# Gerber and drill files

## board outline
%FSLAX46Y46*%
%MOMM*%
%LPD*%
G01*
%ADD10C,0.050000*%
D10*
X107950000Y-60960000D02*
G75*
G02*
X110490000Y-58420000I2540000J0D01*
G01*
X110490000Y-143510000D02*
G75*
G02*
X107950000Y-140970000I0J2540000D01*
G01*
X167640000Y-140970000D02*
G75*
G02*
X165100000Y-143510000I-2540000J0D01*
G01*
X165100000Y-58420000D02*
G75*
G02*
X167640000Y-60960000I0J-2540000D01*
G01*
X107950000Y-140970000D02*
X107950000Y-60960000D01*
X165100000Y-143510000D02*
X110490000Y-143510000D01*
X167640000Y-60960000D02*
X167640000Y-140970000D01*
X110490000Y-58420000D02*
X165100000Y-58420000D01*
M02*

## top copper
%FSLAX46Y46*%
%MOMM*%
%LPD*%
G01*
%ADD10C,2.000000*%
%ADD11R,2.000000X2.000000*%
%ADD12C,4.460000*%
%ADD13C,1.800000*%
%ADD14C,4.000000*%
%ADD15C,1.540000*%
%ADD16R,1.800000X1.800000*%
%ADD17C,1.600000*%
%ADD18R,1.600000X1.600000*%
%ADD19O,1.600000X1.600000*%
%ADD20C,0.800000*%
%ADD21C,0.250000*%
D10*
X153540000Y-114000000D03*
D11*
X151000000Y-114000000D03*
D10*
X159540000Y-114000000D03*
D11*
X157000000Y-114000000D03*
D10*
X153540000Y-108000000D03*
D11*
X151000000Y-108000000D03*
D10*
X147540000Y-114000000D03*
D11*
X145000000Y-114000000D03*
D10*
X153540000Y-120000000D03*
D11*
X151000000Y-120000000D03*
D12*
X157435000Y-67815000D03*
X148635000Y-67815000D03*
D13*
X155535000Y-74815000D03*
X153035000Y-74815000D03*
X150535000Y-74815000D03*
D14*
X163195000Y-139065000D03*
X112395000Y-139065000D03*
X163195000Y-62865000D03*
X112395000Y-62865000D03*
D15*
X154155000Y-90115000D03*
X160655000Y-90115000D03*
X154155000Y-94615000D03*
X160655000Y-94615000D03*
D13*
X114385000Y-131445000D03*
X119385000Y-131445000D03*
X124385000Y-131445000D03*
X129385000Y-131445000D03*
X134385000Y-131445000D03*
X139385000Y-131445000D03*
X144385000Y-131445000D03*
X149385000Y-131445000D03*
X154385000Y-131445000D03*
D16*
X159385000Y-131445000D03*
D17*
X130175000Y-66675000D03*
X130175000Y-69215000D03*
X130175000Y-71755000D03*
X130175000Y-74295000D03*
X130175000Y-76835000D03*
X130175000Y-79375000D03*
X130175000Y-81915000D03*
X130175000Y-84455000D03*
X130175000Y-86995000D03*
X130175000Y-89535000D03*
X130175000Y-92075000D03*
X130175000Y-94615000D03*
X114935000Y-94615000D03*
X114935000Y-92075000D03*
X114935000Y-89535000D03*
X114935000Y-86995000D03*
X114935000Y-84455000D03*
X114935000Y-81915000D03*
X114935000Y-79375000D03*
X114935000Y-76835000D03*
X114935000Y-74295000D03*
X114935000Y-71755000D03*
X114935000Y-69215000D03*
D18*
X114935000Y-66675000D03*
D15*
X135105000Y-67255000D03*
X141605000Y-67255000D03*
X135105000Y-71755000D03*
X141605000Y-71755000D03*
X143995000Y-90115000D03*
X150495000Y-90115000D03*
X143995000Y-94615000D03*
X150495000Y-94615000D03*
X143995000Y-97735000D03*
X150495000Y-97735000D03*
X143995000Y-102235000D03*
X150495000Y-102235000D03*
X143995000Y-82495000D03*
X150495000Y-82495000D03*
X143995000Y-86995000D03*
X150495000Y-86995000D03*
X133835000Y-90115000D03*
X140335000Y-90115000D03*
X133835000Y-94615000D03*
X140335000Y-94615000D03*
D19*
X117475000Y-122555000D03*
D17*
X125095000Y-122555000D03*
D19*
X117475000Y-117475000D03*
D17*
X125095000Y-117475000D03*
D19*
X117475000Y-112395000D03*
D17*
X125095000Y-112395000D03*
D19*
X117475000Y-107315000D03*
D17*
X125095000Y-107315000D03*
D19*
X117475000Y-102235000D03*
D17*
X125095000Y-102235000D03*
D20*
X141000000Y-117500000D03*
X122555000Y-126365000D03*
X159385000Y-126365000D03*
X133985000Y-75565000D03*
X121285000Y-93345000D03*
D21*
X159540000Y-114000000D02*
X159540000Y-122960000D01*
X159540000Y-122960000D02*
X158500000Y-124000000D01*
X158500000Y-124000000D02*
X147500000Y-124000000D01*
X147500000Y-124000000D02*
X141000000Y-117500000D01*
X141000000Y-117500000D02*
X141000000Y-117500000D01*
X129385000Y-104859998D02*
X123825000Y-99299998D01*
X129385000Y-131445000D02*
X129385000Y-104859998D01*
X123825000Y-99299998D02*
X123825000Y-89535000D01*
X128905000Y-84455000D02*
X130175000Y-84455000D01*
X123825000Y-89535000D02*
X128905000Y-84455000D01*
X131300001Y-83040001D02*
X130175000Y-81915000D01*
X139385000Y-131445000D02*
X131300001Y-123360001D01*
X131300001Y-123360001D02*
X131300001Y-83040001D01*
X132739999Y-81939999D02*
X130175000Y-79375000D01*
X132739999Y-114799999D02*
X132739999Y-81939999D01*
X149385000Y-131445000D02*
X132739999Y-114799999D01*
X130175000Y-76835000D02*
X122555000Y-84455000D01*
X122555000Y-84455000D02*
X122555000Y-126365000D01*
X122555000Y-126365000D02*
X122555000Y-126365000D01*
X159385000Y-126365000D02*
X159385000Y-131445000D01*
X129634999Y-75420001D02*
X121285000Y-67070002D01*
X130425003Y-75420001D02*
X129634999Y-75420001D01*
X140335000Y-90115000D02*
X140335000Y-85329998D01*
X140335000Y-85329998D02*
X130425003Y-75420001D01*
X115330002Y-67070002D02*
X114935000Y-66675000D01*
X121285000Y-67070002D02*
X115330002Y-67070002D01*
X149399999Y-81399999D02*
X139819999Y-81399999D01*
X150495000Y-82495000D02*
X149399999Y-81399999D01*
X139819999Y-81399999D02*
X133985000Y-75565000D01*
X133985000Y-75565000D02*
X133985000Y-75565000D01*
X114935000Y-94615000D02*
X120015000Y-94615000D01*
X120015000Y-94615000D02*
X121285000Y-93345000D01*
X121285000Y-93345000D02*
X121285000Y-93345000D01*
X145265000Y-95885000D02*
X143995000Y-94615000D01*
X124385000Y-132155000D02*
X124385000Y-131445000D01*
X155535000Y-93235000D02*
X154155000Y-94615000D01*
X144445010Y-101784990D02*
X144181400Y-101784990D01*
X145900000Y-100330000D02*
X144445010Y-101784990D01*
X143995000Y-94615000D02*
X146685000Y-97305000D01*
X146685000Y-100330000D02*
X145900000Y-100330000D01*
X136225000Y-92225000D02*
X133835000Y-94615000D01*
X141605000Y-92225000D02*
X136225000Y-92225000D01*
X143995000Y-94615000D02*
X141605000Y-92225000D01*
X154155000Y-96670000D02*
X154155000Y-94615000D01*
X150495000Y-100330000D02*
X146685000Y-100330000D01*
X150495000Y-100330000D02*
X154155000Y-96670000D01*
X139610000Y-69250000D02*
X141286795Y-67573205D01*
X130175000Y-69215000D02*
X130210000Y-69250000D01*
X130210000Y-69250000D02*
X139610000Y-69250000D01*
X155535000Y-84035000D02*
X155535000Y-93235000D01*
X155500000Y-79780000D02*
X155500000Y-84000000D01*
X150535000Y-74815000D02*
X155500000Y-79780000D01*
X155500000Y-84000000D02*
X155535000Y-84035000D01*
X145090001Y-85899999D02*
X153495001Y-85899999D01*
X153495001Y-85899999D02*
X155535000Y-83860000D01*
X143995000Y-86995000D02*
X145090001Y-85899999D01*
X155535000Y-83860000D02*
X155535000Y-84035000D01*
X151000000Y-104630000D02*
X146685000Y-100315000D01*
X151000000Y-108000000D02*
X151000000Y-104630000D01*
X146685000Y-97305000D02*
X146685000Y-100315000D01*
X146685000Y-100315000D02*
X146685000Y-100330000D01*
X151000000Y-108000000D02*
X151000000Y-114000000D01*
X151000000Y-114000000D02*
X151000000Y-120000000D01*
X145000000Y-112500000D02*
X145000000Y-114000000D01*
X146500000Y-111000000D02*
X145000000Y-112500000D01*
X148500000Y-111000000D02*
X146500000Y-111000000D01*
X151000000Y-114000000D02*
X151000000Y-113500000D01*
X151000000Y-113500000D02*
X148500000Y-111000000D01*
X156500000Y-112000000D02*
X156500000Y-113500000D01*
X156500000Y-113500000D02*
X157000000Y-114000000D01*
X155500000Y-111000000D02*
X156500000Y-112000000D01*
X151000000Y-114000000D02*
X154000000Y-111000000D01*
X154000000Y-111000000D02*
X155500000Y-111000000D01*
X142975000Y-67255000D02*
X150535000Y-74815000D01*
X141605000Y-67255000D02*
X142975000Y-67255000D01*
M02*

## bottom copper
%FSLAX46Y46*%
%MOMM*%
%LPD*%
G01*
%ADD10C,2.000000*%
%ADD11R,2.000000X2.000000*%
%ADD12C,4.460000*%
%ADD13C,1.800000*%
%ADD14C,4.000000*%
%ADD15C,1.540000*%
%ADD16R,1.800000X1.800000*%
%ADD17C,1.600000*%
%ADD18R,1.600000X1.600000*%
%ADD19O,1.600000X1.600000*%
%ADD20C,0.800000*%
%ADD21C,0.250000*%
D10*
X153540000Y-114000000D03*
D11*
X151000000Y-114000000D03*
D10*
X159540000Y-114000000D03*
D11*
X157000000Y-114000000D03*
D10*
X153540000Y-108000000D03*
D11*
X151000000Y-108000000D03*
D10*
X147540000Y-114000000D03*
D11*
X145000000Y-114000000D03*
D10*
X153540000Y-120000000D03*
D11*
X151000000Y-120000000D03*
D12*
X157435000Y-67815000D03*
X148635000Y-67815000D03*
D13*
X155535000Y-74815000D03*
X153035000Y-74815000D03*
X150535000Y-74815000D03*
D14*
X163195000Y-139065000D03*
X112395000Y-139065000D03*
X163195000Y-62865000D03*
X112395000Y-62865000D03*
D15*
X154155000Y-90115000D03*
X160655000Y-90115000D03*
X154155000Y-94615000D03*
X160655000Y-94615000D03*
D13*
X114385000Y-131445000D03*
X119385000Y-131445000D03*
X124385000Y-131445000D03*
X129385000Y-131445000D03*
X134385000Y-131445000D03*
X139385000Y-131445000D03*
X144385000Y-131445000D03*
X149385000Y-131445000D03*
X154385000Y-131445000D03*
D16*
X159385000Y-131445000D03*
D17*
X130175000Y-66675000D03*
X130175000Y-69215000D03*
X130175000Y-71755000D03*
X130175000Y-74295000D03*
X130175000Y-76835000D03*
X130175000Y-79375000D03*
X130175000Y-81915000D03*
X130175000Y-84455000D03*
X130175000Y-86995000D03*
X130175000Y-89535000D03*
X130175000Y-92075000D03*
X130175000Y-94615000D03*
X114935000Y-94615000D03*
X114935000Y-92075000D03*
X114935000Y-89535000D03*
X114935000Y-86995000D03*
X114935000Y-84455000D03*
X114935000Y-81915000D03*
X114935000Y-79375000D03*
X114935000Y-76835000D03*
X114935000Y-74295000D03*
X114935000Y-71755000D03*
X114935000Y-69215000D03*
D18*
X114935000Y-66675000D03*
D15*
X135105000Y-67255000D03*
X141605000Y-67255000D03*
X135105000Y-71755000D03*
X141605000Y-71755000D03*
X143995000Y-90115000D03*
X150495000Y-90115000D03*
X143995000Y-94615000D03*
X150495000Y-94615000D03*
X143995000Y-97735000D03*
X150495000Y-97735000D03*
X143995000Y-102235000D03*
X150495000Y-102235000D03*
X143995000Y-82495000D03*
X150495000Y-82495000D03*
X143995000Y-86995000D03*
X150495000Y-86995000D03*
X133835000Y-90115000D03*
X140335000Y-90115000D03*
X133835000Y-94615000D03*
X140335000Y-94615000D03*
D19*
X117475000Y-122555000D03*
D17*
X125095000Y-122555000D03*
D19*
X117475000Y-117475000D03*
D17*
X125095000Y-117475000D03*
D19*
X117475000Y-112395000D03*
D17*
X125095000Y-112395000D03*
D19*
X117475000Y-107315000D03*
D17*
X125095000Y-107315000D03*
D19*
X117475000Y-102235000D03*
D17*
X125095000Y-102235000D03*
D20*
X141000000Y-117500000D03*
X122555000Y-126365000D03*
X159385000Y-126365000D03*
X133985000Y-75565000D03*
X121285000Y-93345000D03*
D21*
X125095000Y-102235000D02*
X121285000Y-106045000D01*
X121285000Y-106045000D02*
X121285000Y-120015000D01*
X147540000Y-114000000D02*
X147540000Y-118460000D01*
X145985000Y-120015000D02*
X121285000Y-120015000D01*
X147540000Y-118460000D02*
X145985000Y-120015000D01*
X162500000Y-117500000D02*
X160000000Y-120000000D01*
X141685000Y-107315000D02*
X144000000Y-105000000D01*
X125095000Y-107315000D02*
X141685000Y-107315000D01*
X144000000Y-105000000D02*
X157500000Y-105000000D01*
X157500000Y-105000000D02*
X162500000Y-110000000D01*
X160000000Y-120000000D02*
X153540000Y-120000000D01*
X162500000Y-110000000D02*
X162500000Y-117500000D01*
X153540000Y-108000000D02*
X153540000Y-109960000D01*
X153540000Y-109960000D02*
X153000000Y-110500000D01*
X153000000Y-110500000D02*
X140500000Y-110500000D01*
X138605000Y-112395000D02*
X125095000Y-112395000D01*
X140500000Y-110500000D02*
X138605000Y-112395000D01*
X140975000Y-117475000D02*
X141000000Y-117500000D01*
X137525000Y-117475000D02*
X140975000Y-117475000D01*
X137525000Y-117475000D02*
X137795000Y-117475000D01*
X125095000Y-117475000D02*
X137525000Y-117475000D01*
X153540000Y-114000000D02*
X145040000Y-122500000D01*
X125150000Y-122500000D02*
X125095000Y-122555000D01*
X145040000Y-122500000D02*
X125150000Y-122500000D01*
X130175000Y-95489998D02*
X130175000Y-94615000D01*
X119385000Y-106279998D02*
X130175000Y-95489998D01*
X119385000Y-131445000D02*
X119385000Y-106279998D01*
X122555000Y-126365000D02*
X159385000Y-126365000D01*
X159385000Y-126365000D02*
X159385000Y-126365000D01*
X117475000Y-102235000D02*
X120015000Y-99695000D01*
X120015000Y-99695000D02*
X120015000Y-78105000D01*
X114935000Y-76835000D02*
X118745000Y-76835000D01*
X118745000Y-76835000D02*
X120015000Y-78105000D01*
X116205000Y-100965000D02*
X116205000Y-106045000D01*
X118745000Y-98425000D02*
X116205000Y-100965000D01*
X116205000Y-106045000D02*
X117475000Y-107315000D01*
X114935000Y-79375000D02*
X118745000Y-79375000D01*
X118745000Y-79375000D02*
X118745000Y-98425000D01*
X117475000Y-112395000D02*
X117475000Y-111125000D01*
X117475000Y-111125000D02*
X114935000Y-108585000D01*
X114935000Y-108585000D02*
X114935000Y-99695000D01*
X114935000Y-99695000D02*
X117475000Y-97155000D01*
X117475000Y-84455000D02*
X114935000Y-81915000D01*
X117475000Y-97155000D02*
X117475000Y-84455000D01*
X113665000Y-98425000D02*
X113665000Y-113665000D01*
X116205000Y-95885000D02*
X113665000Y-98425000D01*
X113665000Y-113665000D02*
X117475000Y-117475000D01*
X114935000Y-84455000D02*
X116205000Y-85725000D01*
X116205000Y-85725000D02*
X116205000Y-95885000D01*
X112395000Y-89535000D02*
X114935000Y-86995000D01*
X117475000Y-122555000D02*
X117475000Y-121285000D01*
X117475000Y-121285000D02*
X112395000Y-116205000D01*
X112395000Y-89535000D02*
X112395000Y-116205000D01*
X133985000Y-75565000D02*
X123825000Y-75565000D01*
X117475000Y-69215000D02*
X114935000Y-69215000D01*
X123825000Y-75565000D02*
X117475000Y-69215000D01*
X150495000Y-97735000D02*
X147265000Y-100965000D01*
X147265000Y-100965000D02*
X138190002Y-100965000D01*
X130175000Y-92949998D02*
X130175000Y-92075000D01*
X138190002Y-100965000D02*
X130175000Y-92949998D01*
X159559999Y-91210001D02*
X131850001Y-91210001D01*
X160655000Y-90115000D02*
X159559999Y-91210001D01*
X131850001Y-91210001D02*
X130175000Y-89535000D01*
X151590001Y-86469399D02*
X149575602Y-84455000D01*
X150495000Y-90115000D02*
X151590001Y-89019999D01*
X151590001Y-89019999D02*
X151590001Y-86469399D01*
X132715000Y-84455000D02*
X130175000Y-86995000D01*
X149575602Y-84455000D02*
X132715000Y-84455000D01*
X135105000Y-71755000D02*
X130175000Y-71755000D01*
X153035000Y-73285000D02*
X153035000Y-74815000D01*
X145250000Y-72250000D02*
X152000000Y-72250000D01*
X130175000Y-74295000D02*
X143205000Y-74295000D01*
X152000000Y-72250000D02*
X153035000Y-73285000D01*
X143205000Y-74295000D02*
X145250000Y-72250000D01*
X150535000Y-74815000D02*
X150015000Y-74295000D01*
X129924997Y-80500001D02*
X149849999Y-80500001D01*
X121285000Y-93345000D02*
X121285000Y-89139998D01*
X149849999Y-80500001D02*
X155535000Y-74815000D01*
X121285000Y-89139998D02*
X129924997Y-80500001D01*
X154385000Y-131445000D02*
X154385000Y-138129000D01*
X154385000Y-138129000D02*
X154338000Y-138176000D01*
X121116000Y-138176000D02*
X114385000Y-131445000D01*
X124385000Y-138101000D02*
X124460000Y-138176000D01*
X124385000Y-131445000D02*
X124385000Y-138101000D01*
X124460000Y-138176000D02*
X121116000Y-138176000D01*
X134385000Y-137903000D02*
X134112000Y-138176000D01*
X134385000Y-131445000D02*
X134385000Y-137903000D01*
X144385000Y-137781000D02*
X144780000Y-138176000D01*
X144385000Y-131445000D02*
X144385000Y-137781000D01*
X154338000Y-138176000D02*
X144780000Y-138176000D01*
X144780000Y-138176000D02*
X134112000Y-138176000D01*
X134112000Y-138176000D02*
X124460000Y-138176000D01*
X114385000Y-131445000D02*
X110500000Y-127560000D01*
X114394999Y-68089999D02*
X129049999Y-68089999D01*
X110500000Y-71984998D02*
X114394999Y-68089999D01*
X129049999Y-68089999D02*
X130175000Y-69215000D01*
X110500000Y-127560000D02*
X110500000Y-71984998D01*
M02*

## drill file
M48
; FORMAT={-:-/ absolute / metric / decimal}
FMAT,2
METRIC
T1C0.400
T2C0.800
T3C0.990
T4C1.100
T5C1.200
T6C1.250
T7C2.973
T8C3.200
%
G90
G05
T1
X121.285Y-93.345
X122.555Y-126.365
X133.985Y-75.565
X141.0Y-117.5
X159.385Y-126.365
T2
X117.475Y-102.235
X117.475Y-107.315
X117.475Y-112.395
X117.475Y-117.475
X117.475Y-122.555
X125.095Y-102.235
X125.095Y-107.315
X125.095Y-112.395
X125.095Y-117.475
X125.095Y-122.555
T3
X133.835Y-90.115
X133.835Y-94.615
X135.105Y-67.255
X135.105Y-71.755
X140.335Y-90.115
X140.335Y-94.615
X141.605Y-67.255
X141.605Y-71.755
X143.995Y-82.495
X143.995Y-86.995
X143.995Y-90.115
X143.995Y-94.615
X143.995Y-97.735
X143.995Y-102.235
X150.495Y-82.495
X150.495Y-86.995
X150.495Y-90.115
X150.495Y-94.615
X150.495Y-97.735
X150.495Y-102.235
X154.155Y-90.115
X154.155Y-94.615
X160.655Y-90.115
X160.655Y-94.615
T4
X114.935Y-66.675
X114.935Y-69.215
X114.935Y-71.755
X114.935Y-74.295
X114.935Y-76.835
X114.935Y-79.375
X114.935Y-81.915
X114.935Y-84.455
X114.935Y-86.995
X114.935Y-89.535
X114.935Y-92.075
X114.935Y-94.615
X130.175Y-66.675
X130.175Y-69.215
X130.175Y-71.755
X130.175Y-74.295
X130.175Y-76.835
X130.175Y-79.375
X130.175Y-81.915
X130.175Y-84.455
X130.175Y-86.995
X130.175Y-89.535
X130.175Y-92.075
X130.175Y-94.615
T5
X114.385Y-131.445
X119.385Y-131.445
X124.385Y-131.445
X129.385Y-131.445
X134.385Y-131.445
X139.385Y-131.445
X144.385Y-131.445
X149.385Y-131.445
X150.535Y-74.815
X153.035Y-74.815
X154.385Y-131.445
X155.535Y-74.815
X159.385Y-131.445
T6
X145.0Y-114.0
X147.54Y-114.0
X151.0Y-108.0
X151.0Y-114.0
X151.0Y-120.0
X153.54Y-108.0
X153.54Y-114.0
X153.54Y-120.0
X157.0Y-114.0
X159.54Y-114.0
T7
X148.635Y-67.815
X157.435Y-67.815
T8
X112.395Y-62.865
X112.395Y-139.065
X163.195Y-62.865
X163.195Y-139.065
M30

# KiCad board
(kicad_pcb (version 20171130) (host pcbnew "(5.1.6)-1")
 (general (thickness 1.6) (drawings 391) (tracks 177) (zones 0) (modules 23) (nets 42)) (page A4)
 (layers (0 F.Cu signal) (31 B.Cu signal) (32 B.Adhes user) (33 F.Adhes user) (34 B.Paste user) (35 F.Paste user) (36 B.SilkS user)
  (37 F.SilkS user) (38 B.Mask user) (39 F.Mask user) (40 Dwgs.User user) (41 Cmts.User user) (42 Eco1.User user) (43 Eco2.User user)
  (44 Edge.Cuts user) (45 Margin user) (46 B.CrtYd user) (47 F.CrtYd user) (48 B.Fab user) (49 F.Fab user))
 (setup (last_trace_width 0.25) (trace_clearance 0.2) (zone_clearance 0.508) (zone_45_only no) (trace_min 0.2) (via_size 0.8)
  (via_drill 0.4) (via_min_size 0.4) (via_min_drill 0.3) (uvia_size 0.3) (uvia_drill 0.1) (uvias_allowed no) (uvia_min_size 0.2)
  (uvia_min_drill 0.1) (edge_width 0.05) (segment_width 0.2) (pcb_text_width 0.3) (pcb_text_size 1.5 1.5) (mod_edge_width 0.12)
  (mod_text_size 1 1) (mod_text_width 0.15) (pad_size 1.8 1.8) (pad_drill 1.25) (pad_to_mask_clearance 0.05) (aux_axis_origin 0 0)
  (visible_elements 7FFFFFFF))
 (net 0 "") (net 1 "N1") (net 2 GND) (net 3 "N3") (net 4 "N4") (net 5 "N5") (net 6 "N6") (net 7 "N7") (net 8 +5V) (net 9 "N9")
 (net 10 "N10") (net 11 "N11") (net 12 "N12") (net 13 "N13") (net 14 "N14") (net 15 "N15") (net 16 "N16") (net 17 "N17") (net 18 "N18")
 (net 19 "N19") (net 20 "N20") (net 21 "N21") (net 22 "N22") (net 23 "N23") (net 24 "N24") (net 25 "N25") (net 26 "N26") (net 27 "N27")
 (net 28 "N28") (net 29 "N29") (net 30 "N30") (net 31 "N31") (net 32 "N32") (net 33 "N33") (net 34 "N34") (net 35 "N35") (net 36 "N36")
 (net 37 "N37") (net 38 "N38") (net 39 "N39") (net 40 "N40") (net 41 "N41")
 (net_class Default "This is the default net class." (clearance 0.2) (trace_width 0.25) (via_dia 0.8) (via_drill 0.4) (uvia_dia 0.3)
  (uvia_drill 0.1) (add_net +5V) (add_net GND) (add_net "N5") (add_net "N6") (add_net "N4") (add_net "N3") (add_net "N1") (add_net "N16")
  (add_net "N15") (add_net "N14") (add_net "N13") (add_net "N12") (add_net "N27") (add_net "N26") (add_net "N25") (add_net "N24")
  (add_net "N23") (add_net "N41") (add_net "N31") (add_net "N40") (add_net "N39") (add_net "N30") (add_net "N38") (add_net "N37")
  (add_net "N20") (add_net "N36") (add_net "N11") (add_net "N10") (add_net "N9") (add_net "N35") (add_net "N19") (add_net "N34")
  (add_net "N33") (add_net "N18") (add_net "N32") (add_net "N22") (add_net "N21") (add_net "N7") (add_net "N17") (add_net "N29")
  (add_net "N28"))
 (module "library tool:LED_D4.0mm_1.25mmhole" (layer F.Cu) (at 151 114)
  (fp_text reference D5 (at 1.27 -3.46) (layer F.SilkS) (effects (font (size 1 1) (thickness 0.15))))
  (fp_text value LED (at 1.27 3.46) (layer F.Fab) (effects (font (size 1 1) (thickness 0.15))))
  (pad 2 thru_hole circle (at 2.54 0) (size 2 2) (drill 1.25) (layers *.Cu *.Mask) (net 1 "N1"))
  (pad 1 thru_hole rect (at 0 0) (size 2 2) (drill 1.25) (layers *.Cu *.Mask) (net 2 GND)))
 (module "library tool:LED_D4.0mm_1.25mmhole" (layer F.Cu) (at 157 114)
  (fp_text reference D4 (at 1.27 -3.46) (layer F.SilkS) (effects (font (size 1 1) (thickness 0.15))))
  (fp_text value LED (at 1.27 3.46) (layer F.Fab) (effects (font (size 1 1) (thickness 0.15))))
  (pad 2 thru_hole circle (at 2.54 0) (size 2 2) (drill 1.25) (layers *.Cu *.Mask) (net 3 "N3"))
  (pad 1 thru_hole rect (at 0 0) (size 2 2) (drill 1.25) (layers *.Cu *.Mask) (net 2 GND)))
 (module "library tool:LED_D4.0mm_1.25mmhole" (layer F.Cu) (at 151 108)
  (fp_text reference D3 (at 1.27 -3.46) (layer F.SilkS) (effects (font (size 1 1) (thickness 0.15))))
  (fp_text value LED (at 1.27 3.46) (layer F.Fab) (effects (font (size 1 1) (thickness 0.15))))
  (pad 2 thru_hole circle (at 2.54 0) (size 2 2) (drill 1.25) (layers *.Cu *.Mask) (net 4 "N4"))
  (pad 1 thru_hole rect (at 0 0) (size 2 2) (drill 1.25) (layers *.Cu *.Mask) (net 2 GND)))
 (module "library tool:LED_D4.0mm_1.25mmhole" (layer F.Cu) (at 145 114)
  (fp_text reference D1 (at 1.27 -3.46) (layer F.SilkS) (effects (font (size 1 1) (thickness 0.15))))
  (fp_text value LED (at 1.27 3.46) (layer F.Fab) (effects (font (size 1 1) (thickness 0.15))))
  (pad 2 thru_hole circle (at 2.54 0) (size 2 2) (drill 1.25) (layers *.Cu *.Mask) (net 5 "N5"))
  (pad 1 thru_hole rect (at 0 0) (size 2 2) (drill 1.25) (layers *.Cu *.Mask) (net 2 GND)))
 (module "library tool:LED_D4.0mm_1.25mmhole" (layer F.Cu) (at 151 120)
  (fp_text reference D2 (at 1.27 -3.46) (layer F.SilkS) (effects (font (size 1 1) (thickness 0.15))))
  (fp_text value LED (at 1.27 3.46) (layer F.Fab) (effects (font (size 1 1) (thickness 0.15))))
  (pad 2 thru_hole circle (at 2.54 0) (size 2 2) (drill 1.25) (layers *.Cu *.Mask) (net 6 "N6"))
  (pad 1 thru_hole rect (at 0 0) (size 2 2) (drill 1.25) (layers *.Cu *.Mask) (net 2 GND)))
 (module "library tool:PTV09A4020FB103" (layer F.Cu) (at 153.035 69.215)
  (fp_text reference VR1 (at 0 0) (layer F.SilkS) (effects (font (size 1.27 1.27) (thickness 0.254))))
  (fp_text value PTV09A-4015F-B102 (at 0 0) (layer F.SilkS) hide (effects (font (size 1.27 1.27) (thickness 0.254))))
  (pad 5 thru_hole circle (at 4.4 -1.4) (size 4.46 4.46) (drill 2.9732) (layers *.Cu *.Mask))
  (pad 4 thru_hole circle (at -4.4 -1.4) (size 4.46 4.46) (drill 2.9732) (layers *.Cu *.Mask))
  (pad 3 thru_hole circle (at 2.5 5.6) (size 1.8 1.8) (drill 1.2) (layers *.Cu *.Mask) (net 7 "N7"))
  (pad 2 thru_hole circle (at 0 5.6) (size 1.8 1.8) (drill 1.2) (layers *.Cu *.Mask) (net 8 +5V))
  (pad 1 thru_hole circle (at -2.5 5.6) (size 1.8 1.8) (drill 1.2) (layers *.Cu *.Mask) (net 2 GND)))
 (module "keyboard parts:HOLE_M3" (layer F.Cu) (at 163.195 139.065 180)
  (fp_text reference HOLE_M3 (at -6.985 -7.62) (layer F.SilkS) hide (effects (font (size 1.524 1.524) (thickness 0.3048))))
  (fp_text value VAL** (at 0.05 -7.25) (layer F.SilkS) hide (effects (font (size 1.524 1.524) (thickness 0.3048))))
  (pad 1 thru_hole circle (at 0 0 180) (size 4 4) (drill 3.2) (layers *.Cu *.Mask F.SilkS)))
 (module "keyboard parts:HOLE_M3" (layer F.Cu) (at 112.395 139.065 90)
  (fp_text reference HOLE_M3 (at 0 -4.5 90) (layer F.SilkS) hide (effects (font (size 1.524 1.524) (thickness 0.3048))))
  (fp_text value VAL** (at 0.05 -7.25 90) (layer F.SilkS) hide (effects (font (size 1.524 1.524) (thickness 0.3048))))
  (pad 1 thru_hole circle (at 0 0 90) (size 4 4) (drill 3.2) (layers *.Cu *.Mask F.SilkS)))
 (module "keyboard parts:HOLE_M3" (layer F.Cu) (at 163.195 62.865 270)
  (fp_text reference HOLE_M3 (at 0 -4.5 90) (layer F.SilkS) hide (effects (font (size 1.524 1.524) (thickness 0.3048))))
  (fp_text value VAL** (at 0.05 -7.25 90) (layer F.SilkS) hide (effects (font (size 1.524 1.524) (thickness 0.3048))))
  (pad 1 thru_hole circle (at 0 0 270) (size 4 4) (drill 3.2) (layers *.Cu *.Mask F.SilkS)))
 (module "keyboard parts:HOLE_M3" (layer F.Cu) (at 112.395 62.865)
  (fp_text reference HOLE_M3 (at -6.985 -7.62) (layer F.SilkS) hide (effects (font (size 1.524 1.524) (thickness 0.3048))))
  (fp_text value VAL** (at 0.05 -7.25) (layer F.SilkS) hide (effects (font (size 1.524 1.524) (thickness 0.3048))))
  (pad 1 thru_hole circle (at 0 0) (size 4 4) (drill 3.2) (layers *.Cu *.Mask F.SilkS)))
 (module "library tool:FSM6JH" (layer F.Cu) (at 160.655 94.615)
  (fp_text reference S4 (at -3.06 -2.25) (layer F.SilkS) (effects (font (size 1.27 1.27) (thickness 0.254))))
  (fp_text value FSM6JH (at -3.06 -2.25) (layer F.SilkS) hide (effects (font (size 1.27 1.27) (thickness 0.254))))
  (pad 4 thru_hole circle (at -6.5 -4.5) (size 1.54 1.54) (drill 0.99) (layers *.Cu *.Mask) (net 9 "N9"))
  (pad 3 thru_hole circle (at 0 -4.5) (size 1.54 1.54) (drill 0.99) (layers *.Cu *.Mask) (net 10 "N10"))
  (pad 2 thru_hole circle (at -6.5 0) (size 1.54 1.54) (drill 0.99) (layers *.Cu *.Mask) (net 2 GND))
  (pad 1 thru_hole circle (at 0 0) (size 1.54 1.54) (drill 0.99) (layers *.Cu *.Mask) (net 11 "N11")))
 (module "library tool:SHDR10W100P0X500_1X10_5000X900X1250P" (layer F.Cu) (at 159.385 131.445 180)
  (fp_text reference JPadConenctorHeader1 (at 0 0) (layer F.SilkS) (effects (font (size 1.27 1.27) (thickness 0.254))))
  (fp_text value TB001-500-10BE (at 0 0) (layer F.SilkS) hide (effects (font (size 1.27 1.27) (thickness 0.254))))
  (pad 10 thru_hole circle (at 45 0 180) (size 1.8 1.8) (drill 1.2) (layers *.Cu *.Mask) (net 2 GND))
  (pad 9 thru_hole circle (at 40 0 180) (size 1.8 1.8) (drill 1.2) (layers *.Cu *.Mask) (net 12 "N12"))
  (pad 8 thru_hole circle (at 35 0 180) (size 1.8 1.8) (drill 1.2) (layers *.Cu *.Mask) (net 2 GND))
  (pad 7 thru_hole circle (at 30 0 180) (size 1.8 1.8) (drill 1.2) (layers *.Cu *.Mask) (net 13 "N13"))
  (pad 6 thru_hole circle (at 25 0 180) (size 1.8 1.8) (drill 1.2) (layers *.Cu *.Mask) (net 2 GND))
  (pad 5 thru_hole circle (at 20 0 180) (size 1.8 1.8) (drill 1.2) (layers *.Cu *.Mask) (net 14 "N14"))
  (pad 4 thru_hole circle (at 15 0 180) (size 1.8 1.8) (drill 1.2) (layers *.Cu *.Mask) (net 2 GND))
  (pad 3 thru_hole circle (at 10 0 180) (size 1.8 1.8) (drill 1.2) (layers *.Cu *.Mask) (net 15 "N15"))
  (pad 2 thru_hole circle (at 5 0 180) (size 1.8 1.8) (drill 1.2) (layers *.Cu *.Mask) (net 2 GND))
  (pad 1 thru_hole rect (at 0 0 180) (size 1.8 1.8) (drill 1.2) (layers *.Cu *.Mask) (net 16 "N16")))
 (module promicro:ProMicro (layer F.Cu) (at 122.555 80.645 270)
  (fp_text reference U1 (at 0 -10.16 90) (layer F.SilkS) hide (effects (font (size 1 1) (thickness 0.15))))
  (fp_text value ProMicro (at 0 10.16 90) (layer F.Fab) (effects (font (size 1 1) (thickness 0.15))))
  (pad 24 thru_hole circle (at -13.97 -7.62 270) (size 1.6 1.6) (drill 1.1) (layers *.Cu *.Mask F.SilkS) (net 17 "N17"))
  (pad 23 thru_hole circle (at -11.43 -7.62 270) (size 1.6 1.6) (drill 1.1) (layers *.Cu *.Mask F.SilkS) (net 2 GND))
  (pad 22 thru_hole circle (at -8.89 -7.62 270) (size 1.6 1.6) (drill 1.1) (layers *.Cu *.Mask F.SilkS) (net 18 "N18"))
  (pad 21 thru_hole circle (at -6.35 -7.62 270) (size 1.6 1.6) (drill 1.1) (layers *.Cu *.Mask F.SilkS) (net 8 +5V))
  (pad 20 thru_hole circle (at -3.81 -7.62 270) (size 1.6 1.6) (drill 1.1) (layers *.Cu *.Mask F.SilkS) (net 16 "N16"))
  (pad 19 thru_hole circle (at -1.27 -7.62 270) (size 1.6 1.6) (drill 1.1) (layers *.Cu *.Mask F.SilkS) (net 15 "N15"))
  (pad 18 thru_hole circle (at 1.27 -7.62 270) (size 1.6 1.6) (drill 1.1) (layers *.Cu *.Mask F.SilkS) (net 14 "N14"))
  (pad 17 thru_hole circle (at 3.81 -7.62 270) (size 1.6 1.6) (drill 1.1) (layers *.Cu *.Mask F.SilkS) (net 13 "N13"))
  (pad 16 thru_hole circle (at 6.35 -7.62 270) (size 1.6 1.6) (drill 1.1) (layers *.Cu *.Mask F.SilkS) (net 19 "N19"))
  (pad 15 thru_hole circle (at 8.89 -7.62 270) (size 1.6 1.6) (drill 1.1) (layers *.Cu *.Mask F.SilkS) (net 10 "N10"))
  (pad 14 thru_hole circle (at 11.43 -7.62 270) (size 1.6 1.6) (drill 1.1) (layers *.Cu *.Mask F.SilkS) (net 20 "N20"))
  (pad 13 thru_hole circle (at 13.97 -7.62 270) (size 1.6 1.6) (drill 1.1) (layers *.Cu *.Mask F.SilkS) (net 12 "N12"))
  (pad 12 thru_hole circle (at 13.97 7.62 270) (size 1.6 1.6) (drill 1.1) (layers *.Cu *.Mask F.SilkS) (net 7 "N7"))
  (pad 11 thru_hole circle (at 11.43 7.62 270) (size 1.6 1.6) (drill 1.1) (layers *.Cu *.Mask F.SilkS) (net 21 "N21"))
  (pad 10 thru_hole circle (at 8.89 7.62 270) (size 1.6 1.6) (drill 1.1) (layers *.Cu *.Mask F.SilkS) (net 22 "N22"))
  (pad 9 thru_hole circle (at 6.35 7.62 270) (size 1.6 1.6) (drill 1.1) (layers *.Cu *.Mask F.SilkS) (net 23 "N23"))
  (pad 8 thru_hole circle (at 3.81 7.62 270) (size 1.6 1.6) (drill 1.1) (layers *.Cu *.Mask F.SilkS) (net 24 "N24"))
  (pad 7 thru_hole circle (at 1.27 7.62 270) (size 1.6 1.6) (drill 1.1) (layers *.Cu *.Mask F.SilkS) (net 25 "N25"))
  (pad 6 thru_hole circle (at -1.27 7.62 270) (size 1.6 1.6) (drill 1.1) (layers *.Cu *.Mask F.SilkS) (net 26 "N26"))
  (pad 5 thru_hole circle (at -3.81 7.62 270) (size 1.6 1.6) (drill 1.1) (layers *.Cu *.Mask F.SilkS) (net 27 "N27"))
  (pad 4 thru_hole circle (at -6.35 7.62 270) (size 1.6 1.6) (drill 1.1) (layers *.Cu *.Mask F.SilkS) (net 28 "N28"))
  (pad 3 thru_hole circle (at -8.89 7.62 270) (size 1.6 1.6) (drill 1.1) (layers *.Cu *.Mask F.SilkS) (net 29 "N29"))
  (pad 2 thru_hole circle (at -11.43 7.62 270) (size 1.6 1.6) (drill 1.1) (layers *.Cu *.Mask F.SilkS) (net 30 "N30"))
  (pad 1 thru_hole rect (at -13.97 7.62 270) (size 1.6 1.6) (drill 1.1) (layers *.Cu *.Mask F.SilkS) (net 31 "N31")))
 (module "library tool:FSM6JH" (layer F.Cu) (at 141.605 71.755)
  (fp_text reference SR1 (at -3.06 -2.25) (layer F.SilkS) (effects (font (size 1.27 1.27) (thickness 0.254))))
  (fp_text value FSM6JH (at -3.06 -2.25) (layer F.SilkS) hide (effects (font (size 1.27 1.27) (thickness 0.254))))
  (pad 4 thru_hole circle (at -6.5 -4.5) (size 1.54 1.54) (drill 0.99) (layers *.Cu *.Mask) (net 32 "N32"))
  (pad 3 thru_hole circle (at 0 -4.5) (size 1.54 1.54) (drill 0.99) (layers *.Cu *.Mask) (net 2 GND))
  (pad 2 thru_hole circle (at -6.5 0) (size 1.54 1.54) (drill 0.99) (layers *.Cu *.Mask) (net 18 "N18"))
  (pad 1 thru_hole circle (at 0 0) (size 1.54 1.54) (drill 0.99) (layers *.Cu *.Mask) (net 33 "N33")))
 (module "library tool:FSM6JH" (layer F.Cu) (at 150.495 94.615)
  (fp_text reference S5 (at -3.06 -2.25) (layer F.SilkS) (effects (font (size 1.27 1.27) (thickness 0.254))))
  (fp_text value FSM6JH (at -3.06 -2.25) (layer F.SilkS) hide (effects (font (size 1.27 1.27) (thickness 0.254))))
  (pad 4 thru_hole circle (at -6.5 -4.5) (size 1.54 1.54) (drill 0.99) (layers *.Cu *.Mask) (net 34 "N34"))
  (pad 3 thru_hole circle (at 0 -4.5) (size 1.54 1.54) (drill 0.99) (layers *.Cu *.Mask) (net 19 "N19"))
  (pad 2 thru_hole circle (at -6.5 0) (size 1.54 1.54) (drill 0.99) (layers *.Cu *.Mask) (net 2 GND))
  (pad 1 thru_hole circle (at 0 0) (size 1.54 1.54) (drill 0.99) (layers *.Cu *.Mask) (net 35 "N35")))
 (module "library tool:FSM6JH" (layer F.Cu) (at 150.495 102.235)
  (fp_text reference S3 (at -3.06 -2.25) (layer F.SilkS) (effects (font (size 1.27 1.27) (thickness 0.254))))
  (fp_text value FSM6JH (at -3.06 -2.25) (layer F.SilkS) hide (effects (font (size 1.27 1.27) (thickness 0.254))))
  (pad 4 thru_hole circle (at -6.5 -4.5) (size 1.54 1.54) (drill 0.99) (layers *.Cu *.Mask) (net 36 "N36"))
  (pad 3 thru_hole circle (at 0 -4.5) (size 1.54 1.54) (drill 0.99) (layers *.Cu *.Mask) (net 20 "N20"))
  (pad 2 thru_hole circle (at -6.5 0) (size 1.54 1.54) (drill 0.99) (layers *.Cu *.Mask) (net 2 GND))
  (pad 1 thru_hole circle (at 0 0) (size 1.54 1.54) (drill 0.99) (layers *.Cu *.Mask) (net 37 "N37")))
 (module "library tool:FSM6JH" (layer F.Cu) (at 150.495 86.995)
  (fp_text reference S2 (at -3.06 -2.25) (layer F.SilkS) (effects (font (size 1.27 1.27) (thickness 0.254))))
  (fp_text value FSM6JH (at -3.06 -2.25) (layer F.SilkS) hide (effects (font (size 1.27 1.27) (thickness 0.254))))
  (pad 4 thru_hole circle (at -6.5 -4.5) (size 1.54 1.54) (drill 0.99) (layers *.Cu *.Mask) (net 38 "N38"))
  (pad 3 thru_hole circle (at 0 -4.5) (size 1.54 1.54) (drill 0.99) (layers *.Cu *.Mask) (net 30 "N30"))
  (pad 2 thru_hole circle (at -6.5 0) (size 1.54 1.54) (drill 0.99) (layers *.Cu *.Mask) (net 2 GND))
  (pad 1 thru_hole circle (at 0 0) (size 1.54 1.54) (drill 0.99) (layers *.Cu *.Mask) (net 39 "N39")))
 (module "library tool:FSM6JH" (layer F.Cu) (at 140.335 94.615)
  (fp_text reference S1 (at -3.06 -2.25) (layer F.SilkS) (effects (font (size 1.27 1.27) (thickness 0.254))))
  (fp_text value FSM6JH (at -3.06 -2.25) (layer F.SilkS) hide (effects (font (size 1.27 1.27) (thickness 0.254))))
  (pad 4 thru_hole circle (at -6.5 -4.5) (size 1.54 1.54) (drill 0.99) (layers *.Cu *.Mask) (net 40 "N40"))
  (pad 3 thru_hole circle (at 0 -4.5) (size 1.54 1.54) (drill 0.99) (layers *.Cu *.Mask) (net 31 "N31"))
  (pad 2 thru_hole circle (at -6.5 0) (size 1.54 1.54) (drill 0.99) (layers *.Cu *.Mask) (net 2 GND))
  (pad 1 thru_hole circle (at 0 0) (size 1.54 1.54) (drill 0.99) (layers *.Cu *.Mask) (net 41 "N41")))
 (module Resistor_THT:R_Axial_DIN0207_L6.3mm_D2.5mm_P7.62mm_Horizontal (layer F.Cu) (at 125.095 122.555 180)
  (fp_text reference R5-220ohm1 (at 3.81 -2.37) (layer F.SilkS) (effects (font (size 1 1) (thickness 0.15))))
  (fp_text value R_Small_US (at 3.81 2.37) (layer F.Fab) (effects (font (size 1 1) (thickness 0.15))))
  (pad 2 thru_hole oval (at 7.62 0 180) (size 1.6 1.6) (drill 0.8) (layers *.Cu *.Mask) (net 23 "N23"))
  (pad 1 thru_hole circle (at 0 0 180) (size 1.6 1.6) (drill 0.8) (layers *.Cu *.Mask) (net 1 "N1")))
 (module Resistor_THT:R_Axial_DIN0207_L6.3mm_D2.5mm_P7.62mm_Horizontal (layer F.Cu) (at 125.095 117.475 180)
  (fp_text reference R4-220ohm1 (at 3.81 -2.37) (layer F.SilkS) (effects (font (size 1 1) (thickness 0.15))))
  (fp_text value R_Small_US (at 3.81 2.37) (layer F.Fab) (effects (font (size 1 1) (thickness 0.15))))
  (pad 2 thru_hole oval (at 7.62 0 180) (size 1.6 1.6) (drill 0.8) (layers *.Cu *.Mask) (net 24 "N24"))
  (pad 1 thru_hole circle (at 0 0 180) (size 1.6 1.6) (drill 0.8) (layers *.Cu *.Mask) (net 3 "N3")))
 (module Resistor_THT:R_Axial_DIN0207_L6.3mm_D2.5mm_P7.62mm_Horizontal (layer F.Cu) (at 125.095 112.395 180)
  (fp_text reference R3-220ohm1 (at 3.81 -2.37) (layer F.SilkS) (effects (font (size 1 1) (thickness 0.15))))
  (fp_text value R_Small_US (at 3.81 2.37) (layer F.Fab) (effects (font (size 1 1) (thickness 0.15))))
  (pad 2 thru_hole oval (at 7.62 0 180) (size 1.6 1.6) (drill 0.8) (layers *.Cu *.Mask) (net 25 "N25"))
  (pad 1 thru_hole circle (at 0 0 180) (size 1.6 1.6) (drill 0.8) (layers *.Cu *.Mask) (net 4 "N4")))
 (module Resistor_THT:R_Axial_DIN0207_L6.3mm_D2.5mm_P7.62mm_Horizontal (layer F.Cu) (at 125.095 107.315 180)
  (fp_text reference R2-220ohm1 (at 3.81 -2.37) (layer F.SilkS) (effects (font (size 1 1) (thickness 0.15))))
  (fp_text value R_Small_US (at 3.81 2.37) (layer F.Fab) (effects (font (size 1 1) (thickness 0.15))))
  (pad 2 thru_hole oval (at 7.62 0 180) (size 1.6 1.6) (drill 0.8) (layers *.Cu *.Mask) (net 26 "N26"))
  (pad 1 thru_hole circle (at 0 0 180) (size 1.6 1.6) (drill 0.8) (layers *.Cu *.Mask) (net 6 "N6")))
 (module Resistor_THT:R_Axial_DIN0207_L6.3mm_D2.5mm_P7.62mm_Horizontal (layer F.Cu) (at 125.095 102.235 180)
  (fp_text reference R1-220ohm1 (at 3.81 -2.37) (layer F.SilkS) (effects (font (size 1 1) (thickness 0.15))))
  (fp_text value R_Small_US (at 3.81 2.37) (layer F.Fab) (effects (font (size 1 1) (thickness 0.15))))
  (pad 2 thru_hole oval (at 7.62 0 180) (size 1.6 1.6) (drill 0.8) (layers *.Cu *.Mask) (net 27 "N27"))
  (pad 1 thru_hole circle (at 0 0 180) (size 1.6 1.6) (drill 0.8) (layers *.Cu *.Mask) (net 5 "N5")))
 (gr_arc (start 110.49 60.96) (end 110.49 58.42) (angle -90) (layer Edge.Cuts) (width 0.05))
 (gr_arc (start 110.49 140.97) (end 107.95 140.97) (angle -90) (layer Edge.Cuts) (width 0.05))
 (gr_arc (start 165.1 140.97) (end 165.1 143.51) (angle -90) (layer Edge.Cuts) (width 0.05))
 (gr_arc (start 165.1 60.96) (end 167.64 60.96) (angle -90) (layer Edge.Cuts) (width 0.05))
 (gr_line (start 107.95 140.97) (end 107.95 60.96) (layer Edge.Cuts) (width 0.05))
 (gr_line (start 165.1 143.51) (end 110.49 143.51) (layer Edge.Cuts) (width 0.05))
 (gr_line (start 167.64 60.96) (end 167.64 140.97) (layer Edge.Cuts) (width 0.05))
 (gr_line (start 110.49 58.42) (end 165.1 58.42) (layer Edge.Cuts) (width 0.05))
 (segment (start 125.095 102.235) (end 121.285 106.045) (width 0.25) (layer B.Cu) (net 5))
 (segment (start 121.285 106.045) (end 121.285 120.015) (width 0.25) (layer B.Cu) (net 5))
 (segment (start 147.54 114) (end 147.54 118.46) (width 0.25) (layer B.Cu) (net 5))
 (segment (start 145.985 120.015) (end 121.285 120.015) (width 0.25) (layer B.Cu) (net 5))
 (segment (start 147.54 118.46) (end 145.985 120.015) (width 0.25) (layer B.Cu) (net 5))
 (segment (start 162.5 117.5) (end 160 120) (width 0.25) (layer B.Cu) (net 6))
 (segment (start 141.685 107.315) (end 144 105) (width 0.25) (layer B.Cu) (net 6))
 (segment (start 125.095 107.315) (end 141.685 107.315) (width 0.25) (layer B.Cu) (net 6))
 (segment (start 144 105) (end 157.5 105) (width 0.25) (layer B.Cu) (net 6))
 (segment (start 157.5 105) (end 162.5 110) (width 0.25) (layer B.Cu) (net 6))
 (segment (start 160 120) (end 153.54 120) (width 0.25) (layer B.Cu) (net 6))
 (segment (start 162.5 110) (end 162.5 117.5) (width 0.25) (layer B.Cu) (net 6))
 (segment (start 153.54 108) (end 153.54 109.96) (width 0.25) (layer B.Cu) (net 4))
 (segment (start 153.54 109.96) (end 153 110.5) (width 0.25) (layer B.Cu) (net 4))
 (segment (start 153 110.5) (end 140.5 110.5) (width 0.25) (layer B.Cu) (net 4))
 (segment (start 138.605 112.395) (end 125.095 112.395) (width 0.25) (layer B.Cu) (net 4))
 (segment (start 140.5 110.5) (end 138.605 112.395) (width 0.25) (layer B.Cu) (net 4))
 (segment (start 159.54 114) (end 159.54 122.96) (width 0.25) (layer F.Cu) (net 3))
 (segment (start 159.54 122.96) (end 158.5 124) (width 0.25) (layer F.Cu) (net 3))
 (segment (start 158.5 124) (end 147.5 124) (width 0.25) (layer F.Cu) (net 3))
 (segment (start 147.5 124) (end 141 117.5) (width 0.25) (layer F.Cu) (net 3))
 (segment (start 141 117.5) (end 141 117.5) (width 0.25) (layer F.Cu) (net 3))
 (via (at 141 117.5) (size 0.8) (drill 0.4) (layers F.Cu B.Cu) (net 3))
 (segment (start 140.975 117.475) (end 141 117.5) (width 0.25) (layer B.Cu) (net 3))
 (segment (start 137.525 117.475) (end 140.975 117.475) (width 0.25) (layer B.Cu) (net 3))
 (segment (start 137.525 117.475) (end 137.795 117.475) (width 0.25) (layer B.Cu) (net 3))
 (segment (start 125.095 117.475) (end 137.525 117.475) (width 0.25) (layer B.Cu) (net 3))
 (segment (start 153.54 114) (end 145.04 122.5) (width 0.25) (layer B.Cu) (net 1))
 (segment (start 125.15 122.5) (end 125.095 122.555) (width 0.25) (layer B.Cu) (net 1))
 (segment (start 145.04 122.5) (end 125.15 122.5) (width 0.25) (layer B.Cu) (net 1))
 (segment (start 130.175 95.489998) (end 130.175 94.615) (width 0.25) (layer B.Cu) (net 12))
 (segment (start 119.385 106.279998) (end 130.175 95.489998) (width 0.25) (layer B.Cu) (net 12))
 (segment (start 119.385 131.445) (end 119.385 106.279998) (width 0.25) (layer B.Cu) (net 12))
 (segment (start 129.385 104.859998) (end 123.825 99.299998) (width 0.25) (layer F.Cu) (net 13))
 (segment (start 129.385 131.445) (end 129.385 104.859998) (width 0.25) (layer F.Cu) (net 13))
 (segment (start 123.825 99.299998) (end 123.825 89.535) (width 0.25) (layer F.Cu) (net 13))
 (segment (start 128.905 84.455) (end 130.175 84.455) (width 0.25) (layer F.Cu) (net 13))
 (segment (start 123.825 89.535) (end 128.905 84.455) (width 0.25) (layer F.Cu) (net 13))
 (segment (start 131.300001 83.040001) (end 130.175 81.915) (width 0.25) (layer F.Cu) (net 14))
 (segment (start 139.385 131.445) (end 131.300001 123.360001) (width 0.25) (layer F.Cu) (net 14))
 (segment (start 131.300001 123.360001) (end 131.300001 83.040001) (width 0.25) (layer F.Cu) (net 14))
 (segment (start 132.739999 81.939999) (end 130.175 79.375) (width 0.25) (layer F.Cu) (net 15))
 (segment (start 132.739999 114.799999) (end 132.739999 81.939999) (width 0.25) (layer F.Cu) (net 15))
 (segment (start 149.385 131.445) (end 132.739999 114.799999) (width 0.25) (layer F.Cu) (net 15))
 (segment (start 130.175 76.835) (end 122.555 84.455) (width 0.25) (layer F.Cu) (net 16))
 (segment (start 122.555 84.455) (end 122.555 126.365) (width 0.25) (layer F.Cu) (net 16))
 (segment (start 122.555 126.365) (end 122.555 126.365) (width 0.25) (layer F.Cu) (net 16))
 (via (at 122.555 126.365) (size 0.8) (drill 0.4) (layers F.Cu B.Cu) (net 16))
 (segment (start 122.555 126.365) (end 159.385 126.365) (width 0.25) (layer B.Cu) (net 16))
 (segment (start 159.385 126.365) (end 159.385 126.365) (width 0.25) (layer B.Cu) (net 16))
 (via (at 159.385 126.365) (size 0.8) (drill 0.4) (layers F.Cu B.Cu) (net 16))
 (segment (start 159.385 126.365) (end 159.385 131.445) (width 0.25) (layer F.Cu) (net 16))
 (segment (start 117.475 102.235) (end 120.015 99.695) (width 0.25) (layer B.Cu) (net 27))
 (segment (start 120.015 99.695) (end 120.015 78.105) (width 0.25) (layer B.Cu) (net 27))
 (segment (start 114.935 76.835) (end 118.745 76.835) (width 0.25) (layer B.Cu) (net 27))
 (segment (start 118.745 76.835) (end 120.015 78.105) (width 0.25) (layer B.Cu) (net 27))
 (segment (start 116.205 100.965) (end 116.205 106.045) (width 0.25) (layer B.Cu) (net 26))
 (segment (start 118.745 98.425) (end 116.205 100.965) (width 0.25) (layer B.Cu) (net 26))
 (segment (start 116.205 106.045) (end 117.475 107.315) (width 0.25) (layer B.Cu) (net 26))
 (segment (start 114.935 79.375) (end 118.745 79.375) (width 0.25) (layer B.Cu) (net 26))
 (segment (start 118.745 79.375) (end 118.745 98.425) (width 0.25) (layer B.Cu) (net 26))
 (segment (start 117.475 112.395) (end 117.475 111.125) (width 0.25) (layer B.Cu) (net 25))
 (segment (start 117.475 111.125) (end 114.935 108.585) (width 0.25) (layer B.Cu) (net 25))
 (segment (start 114.935 108.585) (end 114.935 99.695) (width 0.25) (layer B.Cu) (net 25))
 (segment (start 114.935 99.695) (end 117.475 97.155) (width 0.25) (layer B.Cu) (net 25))
 (segment (start 117.475 84.455) (end 114.935 81.915) (width 0.25) (layer B.Cu) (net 25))
 (segment (start 117.475 97.155) (end 117.475 84.455) (width 0.25) (layer B.Cu) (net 25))
 (segment (start 113.665 98.425) (end 113.665 113.665) (width 0.25) (layer B.Cu) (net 24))
 (segment (start 116.205 95.885) (end 113.665 98.425) (width 0.25) (layer B.Cu) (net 24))
 (segment (start 113.665 113.665) (end 117.475 117.475) (width 0.25) (layer B.Cu) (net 24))
 (segment (start 114.935 84.455) (end 116.205 85.725) (width 0.25) (layer B.Cu) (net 24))
 (segment (start 116.205 85.725) (end 116.205 95.885) (width 0.25) (layer B.Cu) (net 24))
 (segment (start 112.395 89.535) (end 114.935 86.995) (width 0.25) (layer B.Cu) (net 23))
 (segment (start 117.475 122.555) (end 117.475 121.285) (width 0.25) (layer B.Cu) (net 23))
 (segment (start 117.475 121.285) (end 112.395 116.205) (width 0.25) (layer B.Cu) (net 23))
 (segment (start 112.395 89.535) (end 112.395 116.205) (width 0.25) (layer B.Cu) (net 23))
 (segment (start 129.634999 75.420001) (end 121.285 67.070002) (width 0.25) (layer F.Cu) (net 31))
 (segment (start 130.425003 75.420001) (end 129.634999 75.420001) (width 0.25) (layer F.Cu) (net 31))
 (segment (start 140.335 90.115) (end 140.335 85.329998) (width 0.25) (layer F.Cu) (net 31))
 (segment (start 140.335 85.329998) (end 130.425003 75.420001) (width 0.25) (layer F.Cu) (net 31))
 (segment (start 115.330002 67.070002) (end 114.935 66.675) (width 0.25) (layer F.Cu) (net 31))
 (segment (start 121.285 67.070002) (end 115.330002 67.070002) (width 0.25) (layer F.Cu) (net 31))
 (segment (start 149.399999 81.399999) (end 139.819999 81.399999) (width 0.25) (layer F.Cu) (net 30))
 (segment (start 150.495 82.495) (end 149.399999 81.399999) (width 0.25) (layer F.Cu) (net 30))
 (segment (start 139.819999 81.399999) (end 133.985 75.565) (width 0.25) (layer F.Cu) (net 30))
 (segment (start 133.985 75.565) (end 133.985 75.565) (width 0.25) (layer F.Cu) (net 30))
 (via (at 133.985 75.565) (size 0.8) (drill 0.4) (layers F.Cu B.Cu) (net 30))
 (segment (start 133.985 75.565) (end 123.825 75.565) (width 0.25) (layer B.Cu) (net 30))
 (segment (start 117.475 69.215) (end 114.935 69.215) (width 0.25) (layer B.Cu) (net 30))
 (segment (start 123.825 75.565) (end 117.475 69.215) (width 0.25) (layer B.Cu) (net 30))
 (segment (start 150.495 97.735) (end 147.265 100.965) (width 0.25) (layer B.Cu) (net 20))
 (segment (start 147.265 100.965) (end 138.190002 100.965) (width 0.25) (layer B.Cu) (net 20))
 (segment (start 130.175 92.949998) (end 130.175 92.075) (width 0.25) (layer B.Cu) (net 20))
 (segment (start 138.190002 100.965) (end 130.175 92.949998) (width 0.25) (layer B.Cu) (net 20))
 (segment (start 159.559999 91.210001) (end 131.850001 91.210001) (width 0.25) (layer B.Cu) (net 10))
 (segment (start 160.655 90.115) (end 159.559999 91.210001) (width 0.25) (layer B.Cu) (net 10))
 (segment (start 131.850001 91.210001) (end 130.175 89.535) (width 0.25) (layer B.Cu) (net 10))
 (segment (start 151.590001 86.469399) (end 149.575602 84.455) (width 0.25) (layer B.Cu) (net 19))
 (segment (start 150.495 90.115) (end 151.590001 89.019999) (width 0.25) (layer B.Cu) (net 19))
 (segment (start 151.590001 89.019999) (end 151.590001 86.469399) (width 0.25) (layer B.Cu) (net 19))
 (segment (start 132.715 84.455) (end 130.175 86.995) (width 0.25) (layer B.Cu) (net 19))
 (segment (start 149.575602 84.455) (end 132.715 84.455) (width 0.25) (layer B.Cu) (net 19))
 (segment (start 135.105 71.755) (end 130.175 71.755) (width 0.25) (layer B.Cu) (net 18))
 (segment (start 153.035 73.285) (end 153.035 74.815) (width 0.25) (layer B.Cu) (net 8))
 (segment (start 145.25 72.25) (end 152 72.25) (width 0.25) (layer B.Cu) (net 8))
 (segment (start 130.175 74.295) (end 143.205 74.295) (width 0.25) (layer B.Cu) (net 8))
 (segment (start 152 72.25) (end 153.035 73.285) (width 0.25) (layer B.Cu) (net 8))
 (segment (start 143.205 74.295) (end 145.25 72.25) (width 0.25) (layer B.Cu) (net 8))
 (segment (start 150.535 74.815) (end 150.015 74.295) (width 0.25) (layer B.Cu) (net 2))
 (segment (start 114.935 94.615) (end 120.015 94.615) (width 0.25) (layer F.Cu) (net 7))
 (segment (start 120.015 94.615) (end 121.285 93.345) (width 0.25) (layer F.Cu) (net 7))
 (segment (start 121.285 93.345) (end 121.285 93.345) (width 0.25) (layer F.Cu) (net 7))
 (via (at 121.285 93.345) (size 0.8) (drill 0.4) (layers F.Cu B.Cu) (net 7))
 (segment (start 129.924997 80.500001) (end 149.849999 80.500001) (width 0.25) (layer B.Cu) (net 7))
 (segment (start 121.285 93.345) (end 121.285 89.139998) (width 0.25) (layer B.Cu) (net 7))
 (segment (start 149.849999 80.500001) (end 155.535 74.815) (width 0.25) (layer B.Cu) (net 7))
 (segment (start 121.285 89.139998) (end 129.924997 80.500001) (width 0.25) (layer B.Cu) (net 7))
 (segment (start 145.265 95.885) (end 143.995 94.615) (width 0.25) (layer F.Cu) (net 2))
 (segment (start 124.385 132.155) (end 124.385 131.445) (width 0.25) (layer F.Cu) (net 2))
 (segment (start 155.535 93.235) (end 154.155 94.615) (width 0.25) (layer F.Cu) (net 2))
 (segment (start 144.44501 101.78499) (end 144.1814 101.78499) (width 0.25) (layer F.Cu) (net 2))
 (segment (start 145.9 100.33) (end 144.44501 101.78499) (width 0.25) (layer F.Cu) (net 2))
 (segment (start 143.995 94.615) (end 146.685 97.305) (width 0.25) (layer F.Cu) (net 2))
 (segment (start 146.685 100.33) (end 145.9 100.33) (width 0.25) (layer F.Cu) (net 2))
 (segment (start 136.225 92.225) (end 133.835 94.615) (width 0.25) (layer F.Cu) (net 2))
 (segment (start 141.605 92.225) (end 136.225 92.225) (width 0.25) (layer F.Cu) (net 2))
 (segment (start 143.995 94.615) (end 141.605 92.225) (width 0.25) (layer F.Cu) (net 2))
 (segment (start 154.155 96.67) (end 154.155 94.615) (width 0.25) (layer F.Cu) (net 2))
 (segment (start 150.495 100.33) (end 146.685 100.33) (width 0.25) (layer F.Cu) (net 2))
 (segment (start 150.495 100.33) (end 154.155 96.67) (width 0.25) (layer F.Cu) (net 2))
 (segment (start 154.385 131.445) (end 154.385 138.129) (width 0.25) (layer B.Cu) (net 2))
 (segment (start 154.385 138.129) (end 154.338 138.176) (width 0.25) (layer B.Cu) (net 2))
 (segment (start 121.116 138.176) (end 114.385 131.445) (width 0.25) (layer B.Cu) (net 2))
 (segment (start 124.385 138.101) (end 124.46 138.176) (width 0.25) (layer B.Cu) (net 2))
 (segment (start 124.385 131.445) (end 124.385 138.101) (width 0.25) (layer B.Cu) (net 2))
 (segment (start 124.46 138.176) (end 121.116 138.176) (width 0.25) (layer B.Cu) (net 2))
 (segment (start 134.385 137.903) (end 134.112 138.176) (width 0.25) (layer B.Cu) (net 2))
 (segment (start 134.385 131.445) (end 134.385 137.903) (width 0.25) (layer B.Cu) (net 2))
 (segment (start 144.385 137.781) (end 144.78 138.176) (width 0.25) (layer B.Cu) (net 2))
 (segment (start 144.385 131.445) (end 144.385 137.781) (width 0.25) (layer B.Cu) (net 2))
 (segment (start 154.338 138.176) (end 144.78 138.176) (width 0.25) (layer B.Cu) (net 2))
 (segment (start 144.78 138.176) (end 134.112 138.176) (width 0.25) (layer B.Cu) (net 2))
 (segment (start 139.61 69.25) (end 141.286795 67.573205) (width 0.25) (layer F.Cu) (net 2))
 (segment (start 130.175 69.215) (end 130.21 69.25) (width 0.25) (layer F.Cu) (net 2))
 (segment (start 130.21 69.25) (end 139.61 69.25) (width 0.25) (layer F.Cu) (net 2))
 (segment (start 134.112 138.176) (end 124.46 138.176) (width 0.25) (layer B.Cu) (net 2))
 (segment (start 155.535 84.035) (end 155.535 93.235) (width 0.25) (layer F.Cu) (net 2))
 (segment (start 155.5 79.78) (end 155.5 84) (width 0.25) (layer F.Cu) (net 2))
 (segment (start 150.535 74.815) (end 155.5 79.78) (width 0.25) (layer F.Cu) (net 2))
 (segment (start 155.5 84) (end 155.535 84.035) (width 0.25) (layer F.Cu) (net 2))
 (segment (start 145.090001 85.899999) (end 153.495001 85.899999) (width 0.25) (layer F.Cu) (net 2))
 (segment (start 153.495001 85.899999) (end 155.535 83.86) (width 0.25) (layer F.Cu) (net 2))
 (segment (start 143.995 86.995) (end 145.090001 85.899999) (width 0.25) (layer F.Cu) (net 2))
 (segment (start 155.535 83.86) (end 155.535 84.035) (width 0.25) (layer F.Cu) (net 2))
 (segment (start 151 104.63) (end 146.685 100.315) (width 0.25) (layer F.Cu) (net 2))
 (segment (start 151 108) (end 151 104.63) (width 0.25) (layer F.Cu) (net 2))
 (segment (start 146.685 97.305) (end 146.685 100.315) (width 0.25) (layer F.Cu) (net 2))
 (segment (start 146.685 100.315) (end 146.685 100.33) (width 0.25) (layer F.Cu) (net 2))
 (segment (start 151 108) (end 151 114) (width 0.25) (layer F.Cu) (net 2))
 (segment (start 151 114) (end 151 120) (width 0.25) (layer F.Cu) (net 2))
 (segment (start 145 112.5) (end 145 114) (width 0.25) (layer F.Cu) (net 2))
 (segment (start 146.5 111) (end 145 112.5) (width 0.25) (layer F.Cu) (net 2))
 (segment (start 148.5 111) (end 146.5 111) (width 0.25) (layer F.Cu) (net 2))
 (segment (start 151 114) (end 151 113.5) (width 0.25) (layer F.Cu) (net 2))
 (segment (start 151 113.5) (end 148.5 111) (width 0.25) (layer F.Cu) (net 2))
 (segment (start 156.5 112) (end 156.5 113.5) (width 0.25) (layer F.Cu) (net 2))
 (segment (start 156.5 113.5) (end 157 114) (width 0.25) (layer F.Cu) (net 2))
 (segment (start 155.5 111) (end 156.5 112) (width 0.25) (layer F.Cu) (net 2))
 (segment (start 151 114) (end 154 111) (width 0.25) (layer F.Cu) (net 2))
 (segment (start 154 111) (end 155.5 111) (width 0.25) (layer F.Cu) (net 2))
 (segment (start 114.385 131.445) (end 110.5 127.56) (width 0.25) (layer B.Cu) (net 2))
 (segment (start 114.394999 68.089999) (end 129.049999 68.089999) (width 0.25) (layer B.Cu) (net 2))
 (segment (start 110.5 71.984998) (end 114.394999 68.089999) (width 0.25) (layer B.Cu) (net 2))
 (segment (start 129.049999 68.089999) (end 130.175 69.215) (width 0.25) (layer B.Cu) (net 2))
 (segment (start 110.5 127.56) (end 110.5 71.984998) (width 0.25) (layer B.Cu) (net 2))
 (segment (start 142.975 67.255) (end 150.535 74.815) (width 0.25) (layer F.Cu) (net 2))
 (segment (start 141.605 67.255) (end 142.975 67.255) (width 0.25) (layer F.Cu) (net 2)))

